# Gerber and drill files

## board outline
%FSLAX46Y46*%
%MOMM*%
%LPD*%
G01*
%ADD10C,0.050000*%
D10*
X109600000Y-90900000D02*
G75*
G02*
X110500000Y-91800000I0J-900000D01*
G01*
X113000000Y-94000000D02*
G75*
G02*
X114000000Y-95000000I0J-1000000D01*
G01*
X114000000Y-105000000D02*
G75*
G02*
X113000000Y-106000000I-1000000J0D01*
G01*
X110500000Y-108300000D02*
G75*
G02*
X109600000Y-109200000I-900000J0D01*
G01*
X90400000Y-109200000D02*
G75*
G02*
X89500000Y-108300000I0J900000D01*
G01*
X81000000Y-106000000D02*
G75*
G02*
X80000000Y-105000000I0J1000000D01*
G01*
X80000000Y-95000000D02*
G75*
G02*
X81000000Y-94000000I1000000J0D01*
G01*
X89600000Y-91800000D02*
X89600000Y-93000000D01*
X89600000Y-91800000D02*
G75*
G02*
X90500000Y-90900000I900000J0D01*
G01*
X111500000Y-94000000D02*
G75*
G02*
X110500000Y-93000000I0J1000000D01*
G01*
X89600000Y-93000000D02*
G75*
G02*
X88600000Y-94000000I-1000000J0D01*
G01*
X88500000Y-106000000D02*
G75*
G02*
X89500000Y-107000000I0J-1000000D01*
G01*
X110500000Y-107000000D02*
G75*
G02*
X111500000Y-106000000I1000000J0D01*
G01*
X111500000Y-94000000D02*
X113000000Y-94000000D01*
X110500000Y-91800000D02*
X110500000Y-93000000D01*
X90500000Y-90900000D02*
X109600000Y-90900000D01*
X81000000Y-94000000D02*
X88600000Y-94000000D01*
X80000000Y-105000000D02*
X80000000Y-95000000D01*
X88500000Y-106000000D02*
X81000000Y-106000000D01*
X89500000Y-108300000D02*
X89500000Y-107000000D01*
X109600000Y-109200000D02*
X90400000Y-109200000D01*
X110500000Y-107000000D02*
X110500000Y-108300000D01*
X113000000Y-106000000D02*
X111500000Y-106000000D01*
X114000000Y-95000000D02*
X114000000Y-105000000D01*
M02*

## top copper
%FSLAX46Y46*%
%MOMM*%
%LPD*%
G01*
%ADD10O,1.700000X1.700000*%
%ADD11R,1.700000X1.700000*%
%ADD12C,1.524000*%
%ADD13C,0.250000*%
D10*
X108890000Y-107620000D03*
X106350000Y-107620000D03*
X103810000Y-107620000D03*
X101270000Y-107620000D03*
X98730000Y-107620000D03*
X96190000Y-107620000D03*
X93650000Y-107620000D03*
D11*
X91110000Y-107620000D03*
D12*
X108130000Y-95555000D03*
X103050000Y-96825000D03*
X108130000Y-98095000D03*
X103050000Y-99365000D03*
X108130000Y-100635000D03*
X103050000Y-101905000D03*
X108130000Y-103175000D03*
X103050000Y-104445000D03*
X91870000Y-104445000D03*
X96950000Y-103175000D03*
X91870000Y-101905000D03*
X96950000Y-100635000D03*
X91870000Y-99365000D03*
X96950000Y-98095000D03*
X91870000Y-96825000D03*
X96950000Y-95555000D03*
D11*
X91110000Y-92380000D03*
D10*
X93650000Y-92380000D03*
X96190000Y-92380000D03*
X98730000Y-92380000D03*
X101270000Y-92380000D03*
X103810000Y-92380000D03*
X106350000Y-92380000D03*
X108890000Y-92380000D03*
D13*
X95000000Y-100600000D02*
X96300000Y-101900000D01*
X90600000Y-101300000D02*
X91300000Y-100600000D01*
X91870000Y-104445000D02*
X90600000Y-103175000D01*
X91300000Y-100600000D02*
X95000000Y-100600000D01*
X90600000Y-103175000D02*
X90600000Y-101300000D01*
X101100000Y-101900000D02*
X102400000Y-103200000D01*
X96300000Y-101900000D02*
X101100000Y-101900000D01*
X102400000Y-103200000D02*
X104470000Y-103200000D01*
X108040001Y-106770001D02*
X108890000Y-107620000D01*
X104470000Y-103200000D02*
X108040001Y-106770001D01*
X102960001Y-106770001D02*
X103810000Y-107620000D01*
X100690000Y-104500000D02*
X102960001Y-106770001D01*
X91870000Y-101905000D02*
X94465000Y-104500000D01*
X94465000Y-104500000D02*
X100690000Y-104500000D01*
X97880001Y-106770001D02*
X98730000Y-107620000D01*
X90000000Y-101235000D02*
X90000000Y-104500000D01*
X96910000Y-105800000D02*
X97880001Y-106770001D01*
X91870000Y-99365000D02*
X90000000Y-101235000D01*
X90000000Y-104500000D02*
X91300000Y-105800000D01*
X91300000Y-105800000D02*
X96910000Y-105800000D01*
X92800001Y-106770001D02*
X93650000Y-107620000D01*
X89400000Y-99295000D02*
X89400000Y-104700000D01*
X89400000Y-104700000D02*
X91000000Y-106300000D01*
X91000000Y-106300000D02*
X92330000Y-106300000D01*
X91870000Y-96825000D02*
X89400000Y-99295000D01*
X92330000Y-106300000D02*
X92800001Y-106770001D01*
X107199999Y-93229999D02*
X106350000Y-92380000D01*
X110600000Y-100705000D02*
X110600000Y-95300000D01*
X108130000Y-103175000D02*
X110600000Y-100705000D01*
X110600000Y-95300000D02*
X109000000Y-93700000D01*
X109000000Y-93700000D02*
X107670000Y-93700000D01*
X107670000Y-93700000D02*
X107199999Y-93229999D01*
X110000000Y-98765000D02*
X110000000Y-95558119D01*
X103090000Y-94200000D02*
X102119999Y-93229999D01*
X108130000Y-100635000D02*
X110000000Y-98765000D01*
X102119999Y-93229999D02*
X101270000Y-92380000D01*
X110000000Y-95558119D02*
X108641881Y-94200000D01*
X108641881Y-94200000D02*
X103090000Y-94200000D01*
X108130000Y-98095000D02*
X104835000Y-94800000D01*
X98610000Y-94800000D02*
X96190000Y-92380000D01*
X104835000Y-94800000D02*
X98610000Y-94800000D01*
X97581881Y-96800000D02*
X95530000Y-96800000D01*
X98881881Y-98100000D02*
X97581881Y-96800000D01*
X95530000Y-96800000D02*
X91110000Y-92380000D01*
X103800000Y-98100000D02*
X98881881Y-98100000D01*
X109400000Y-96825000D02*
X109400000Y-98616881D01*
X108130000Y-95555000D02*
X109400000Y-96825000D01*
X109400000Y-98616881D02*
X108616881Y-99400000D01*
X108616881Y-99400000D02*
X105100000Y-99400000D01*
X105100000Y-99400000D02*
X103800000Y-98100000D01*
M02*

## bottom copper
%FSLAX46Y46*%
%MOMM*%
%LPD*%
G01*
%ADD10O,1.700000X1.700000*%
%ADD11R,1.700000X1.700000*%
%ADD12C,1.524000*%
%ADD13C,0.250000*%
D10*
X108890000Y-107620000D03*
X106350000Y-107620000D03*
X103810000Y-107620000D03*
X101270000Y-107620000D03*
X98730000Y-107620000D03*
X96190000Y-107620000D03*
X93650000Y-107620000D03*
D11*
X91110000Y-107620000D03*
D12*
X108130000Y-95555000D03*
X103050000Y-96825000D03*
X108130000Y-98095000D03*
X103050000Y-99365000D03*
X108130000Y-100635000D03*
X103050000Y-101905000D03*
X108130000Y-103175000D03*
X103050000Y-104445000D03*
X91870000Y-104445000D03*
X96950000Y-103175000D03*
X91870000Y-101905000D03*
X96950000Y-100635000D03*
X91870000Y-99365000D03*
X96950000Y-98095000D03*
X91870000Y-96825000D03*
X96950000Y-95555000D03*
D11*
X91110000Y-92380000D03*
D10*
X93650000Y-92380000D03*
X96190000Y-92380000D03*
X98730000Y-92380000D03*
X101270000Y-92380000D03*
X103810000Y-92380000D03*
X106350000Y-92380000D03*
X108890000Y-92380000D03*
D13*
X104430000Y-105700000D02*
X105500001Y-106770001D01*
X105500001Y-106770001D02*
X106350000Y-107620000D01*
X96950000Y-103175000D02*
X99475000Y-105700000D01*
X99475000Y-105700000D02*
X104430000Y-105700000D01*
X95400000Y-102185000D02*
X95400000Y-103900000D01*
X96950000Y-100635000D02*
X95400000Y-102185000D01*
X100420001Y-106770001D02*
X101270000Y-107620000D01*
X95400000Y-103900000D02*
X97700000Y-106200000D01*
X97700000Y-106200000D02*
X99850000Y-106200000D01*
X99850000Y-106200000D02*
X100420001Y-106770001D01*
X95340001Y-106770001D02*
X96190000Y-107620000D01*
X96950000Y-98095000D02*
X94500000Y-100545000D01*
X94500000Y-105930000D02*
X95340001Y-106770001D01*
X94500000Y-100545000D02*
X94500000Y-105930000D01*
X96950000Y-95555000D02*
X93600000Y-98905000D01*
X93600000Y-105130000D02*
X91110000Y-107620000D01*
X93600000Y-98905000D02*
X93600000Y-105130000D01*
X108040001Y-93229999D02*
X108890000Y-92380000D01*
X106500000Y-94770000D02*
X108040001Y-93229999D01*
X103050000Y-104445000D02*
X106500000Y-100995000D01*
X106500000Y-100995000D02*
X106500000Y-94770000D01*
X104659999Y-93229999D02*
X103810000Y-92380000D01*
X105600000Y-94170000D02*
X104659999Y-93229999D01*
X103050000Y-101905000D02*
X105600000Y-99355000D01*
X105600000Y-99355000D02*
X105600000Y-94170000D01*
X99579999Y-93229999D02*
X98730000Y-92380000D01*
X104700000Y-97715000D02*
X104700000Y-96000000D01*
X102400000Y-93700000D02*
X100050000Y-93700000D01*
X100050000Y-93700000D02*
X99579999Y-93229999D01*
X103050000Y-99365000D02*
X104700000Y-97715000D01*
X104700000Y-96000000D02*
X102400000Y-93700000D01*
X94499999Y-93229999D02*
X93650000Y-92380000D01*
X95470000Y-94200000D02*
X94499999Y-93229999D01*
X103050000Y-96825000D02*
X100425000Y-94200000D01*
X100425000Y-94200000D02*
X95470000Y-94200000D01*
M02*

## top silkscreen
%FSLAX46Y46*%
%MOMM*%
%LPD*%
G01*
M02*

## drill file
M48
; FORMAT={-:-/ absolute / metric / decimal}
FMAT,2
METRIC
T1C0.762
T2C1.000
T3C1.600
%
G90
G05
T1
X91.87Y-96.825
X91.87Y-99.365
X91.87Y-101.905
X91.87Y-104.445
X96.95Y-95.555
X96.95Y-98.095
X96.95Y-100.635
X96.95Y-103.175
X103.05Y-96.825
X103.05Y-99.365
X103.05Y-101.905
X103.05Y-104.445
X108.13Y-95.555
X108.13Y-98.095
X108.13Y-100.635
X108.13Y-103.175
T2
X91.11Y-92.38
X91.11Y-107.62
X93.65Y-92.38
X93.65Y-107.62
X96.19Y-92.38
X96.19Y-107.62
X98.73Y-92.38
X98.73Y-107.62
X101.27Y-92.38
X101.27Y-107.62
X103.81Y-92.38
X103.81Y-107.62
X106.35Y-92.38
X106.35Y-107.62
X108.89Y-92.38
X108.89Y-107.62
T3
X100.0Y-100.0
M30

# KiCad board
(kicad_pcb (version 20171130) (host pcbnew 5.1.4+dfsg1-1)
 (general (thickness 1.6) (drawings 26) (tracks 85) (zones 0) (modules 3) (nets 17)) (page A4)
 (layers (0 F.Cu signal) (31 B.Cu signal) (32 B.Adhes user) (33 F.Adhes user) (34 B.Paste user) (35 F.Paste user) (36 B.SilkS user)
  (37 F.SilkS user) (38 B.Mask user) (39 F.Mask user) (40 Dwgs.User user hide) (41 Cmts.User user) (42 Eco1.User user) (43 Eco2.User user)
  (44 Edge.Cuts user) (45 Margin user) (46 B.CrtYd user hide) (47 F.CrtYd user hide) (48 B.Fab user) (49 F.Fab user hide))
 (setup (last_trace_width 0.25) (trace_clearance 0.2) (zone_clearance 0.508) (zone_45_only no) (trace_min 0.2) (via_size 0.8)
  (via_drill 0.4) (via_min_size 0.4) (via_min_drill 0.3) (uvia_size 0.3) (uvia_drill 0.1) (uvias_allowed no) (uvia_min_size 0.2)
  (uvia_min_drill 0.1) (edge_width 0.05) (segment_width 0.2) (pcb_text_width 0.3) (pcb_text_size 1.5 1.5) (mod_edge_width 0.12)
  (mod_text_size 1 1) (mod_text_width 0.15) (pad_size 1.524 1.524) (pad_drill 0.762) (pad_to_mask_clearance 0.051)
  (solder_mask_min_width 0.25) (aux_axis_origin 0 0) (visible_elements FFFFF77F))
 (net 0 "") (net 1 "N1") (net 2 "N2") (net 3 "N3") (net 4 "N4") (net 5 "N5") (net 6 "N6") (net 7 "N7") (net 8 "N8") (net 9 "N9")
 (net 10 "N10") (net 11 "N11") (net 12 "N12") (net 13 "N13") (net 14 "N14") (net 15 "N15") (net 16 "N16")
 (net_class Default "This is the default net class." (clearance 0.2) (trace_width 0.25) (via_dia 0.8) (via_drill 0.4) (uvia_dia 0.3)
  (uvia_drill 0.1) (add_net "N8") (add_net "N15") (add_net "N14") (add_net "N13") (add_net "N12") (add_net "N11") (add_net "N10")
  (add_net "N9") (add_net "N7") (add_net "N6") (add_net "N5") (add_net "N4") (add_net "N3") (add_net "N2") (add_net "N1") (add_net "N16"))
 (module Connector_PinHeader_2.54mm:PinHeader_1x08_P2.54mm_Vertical (layer B.Cu) (at 91.11 107.62 270)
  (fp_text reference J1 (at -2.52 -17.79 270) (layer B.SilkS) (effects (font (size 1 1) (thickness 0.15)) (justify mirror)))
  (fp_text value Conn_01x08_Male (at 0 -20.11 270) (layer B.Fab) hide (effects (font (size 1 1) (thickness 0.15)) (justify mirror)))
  (pad 8 thru_hole oval (at 0 -17.78 270) (size 1.7 1.7) (drill 1) (layers *.Cu *.Mask) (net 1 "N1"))
  (pad 7 thru_hole oval (at 0 -15.24 270) (size 1.7 1.7) (drill 1) (layers *.Cu *.Mask) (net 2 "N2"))
  (pad 6 thru_hole oval (at 0 -12.7 270) (size 1.7 1.7) (drill 1) (layers *.Cu *.Mask) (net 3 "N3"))
  (pad 5 thru_hole oval (at 0 -10.16 270) (size 1.7 1.7) (drill 1) (layers *.Cu *.Mask) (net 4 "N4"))
  (pad 4 thru_hole oval (at 0 -7.62 270) (size 1.7 1.7) (drill 1) (layers *.Cu *.Mask) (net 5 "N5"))
  (pad 3 thru_hole oval (at 0 -5.08 270) (size 1.7 1.7) (drill 1) (layers *.Cu *.Mask) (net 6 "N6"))
  (pad 2 thru_hole oval (at 0 -2.54 270) (size 1.7 1.7) (drill 1) (layers *.Cu *.Mask) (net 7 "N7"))
  (pad 1 thru_hole rect (at 0 0 270) (size 1.7 1.7) (drill 1) (layers *.Cu *.Mask) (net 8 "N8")))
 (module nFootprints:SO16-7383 (layer F.Cu) (at 100 100)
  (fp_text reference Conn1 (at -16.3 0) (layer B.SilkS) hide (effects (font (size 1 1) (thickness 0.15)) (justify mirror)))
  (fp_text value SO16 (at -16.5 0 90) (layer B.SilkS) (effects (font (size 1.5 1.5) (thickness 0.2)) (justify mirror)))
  (pad "" np_thru_hole circle (at 0 0) (size 1.6 1.6) (drill 1.6) (layers *.Cu *.Mask))
  (pad 16 thru_hole circle (at 8.13 -4.445) (size 1.524 1.524) (drill 0.762) (layers *.Cu *.Mask) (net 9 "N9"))
  (pad 15 thru_hole circle (at 3.05 -3.175) (size 1.524 1.524) (drill 0.762) (layers *.Cu *.Mask) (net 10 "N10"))
  (pad 14 thru_hole circle (at 8.13 -1.905) (size 1.524 1.524) (drill 0.762) (layers *.Cu *.Mask) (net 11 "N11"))
  (pad 13 thru_hole circle (at 3.05 -0.635) (size 1.524 1.524) (drill 0.762) (layers *.Cu *.Mask) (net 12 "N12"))
  (pad 12 thru_hole circle (at 8.13 0.635) (size 1.524 1.524) (drill 0.762) (layers *.Cu *.Mask) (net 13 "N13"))
  (pad 11 thru_hole circle (at 3.05 1.905) (size 1.524 1.524) (drill 0.762) (layers *.Cu *.Mask) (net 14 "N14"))
  (pad 10 thru_hole circle (at 8.13 3.175) (size 1.524 1.524) (drill 0.762) (layers *.Cu *.Mask) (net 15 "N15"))
  (pad 9 thru_hole circle (at 3.05 4.445) (size 1.524 1.524) (drill 0.762) (layers *.Cu *.Mask) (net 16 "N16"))
  (pad 8 thru_hole circle (at -8.13 4.445) (size 1.524 1.524) (drill 0.762) (layers *.Cu *.Mask) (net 1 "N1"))
  (pad 7 thru_hole circle (at -3.05 3.175) (size 1.524 1.524) (drill 0.762) (layers *.Cu *.Mask) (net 2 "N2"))
  (pad 6 thru_hole circle (at -8.13 1.905) (size 1.524 1.524) (drill 0.762) (layers *.Cu *.Mask) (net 3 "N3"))
  (pad 5 thru_hole circle (at -3.05 0.635) (size 1.524 1.524) (drill 0.762) (layers *.Cu *.Mask) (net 4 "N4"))
  (pad 4 thru_hole circle (at -8.13 -0.635) (size 1.524 1.524) (drill 0.762) (layers *.Cu *.Mask) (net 5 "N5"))
  (pad 3 thru_hole circle (at -3.05 -1.905) (size 1.524 1.524) (drill 0.762) (layers *.Cu *.Mask) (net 6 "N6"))
  (pad 2 thru_hole circle (at -8.13 -3.175) (size 1.524 1.524) (drill 0.762) (layers *.Cu *.Mask) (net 7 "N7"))
  (pad 1 thru_hole circle (at -3.05 -4.445) (size 1.524 1.524) (drill 0.762) (layers *.Cu *.Mask) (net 8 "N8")))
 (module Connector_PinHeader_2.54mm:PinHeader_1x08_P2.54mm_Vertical (layer B.Cu) (at 91.11 92.38 270)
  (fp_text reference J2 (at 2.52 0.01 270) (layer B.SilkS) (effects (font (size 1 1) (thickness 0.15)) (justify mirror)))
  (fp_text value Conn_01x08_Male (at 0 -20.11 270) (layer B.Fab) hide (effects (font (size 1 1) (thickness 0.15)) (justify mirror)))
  (pad 1 thru_hole rect (at 0 0 270) (size 1.7 1.7) (drill 1) (layers *.Cu *.Mask) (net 9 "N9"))
  (pad 2 thru_hole oval (at 0 -2.54 270) (size 1.7 1.7) (drill 1) (layers *.Cu *.Mask) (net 10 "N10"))
  (pad 3 thru_hole oval (at 0 -5.08 270) (size 1.7 1.7) (drill 1) (layers *.Cu *.Mask) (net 11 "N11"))
  (pad 4 thru_hole oval (at 0 -7.62 270) (size 1.7 1.7) (drill 1) (layers *.Cu *.Mask) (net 12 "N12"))
  (pad 5 thru_hole oval (at 0 -10.16 270) (size 1.7 1.7) (drill 1) (layers *.Cu *.Mask) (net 13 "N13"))
  (pad 6 thru_hole oval (at 0 -12.7 270) (size 1.7 1.7) (drill 1) (layers *.Cu *.Mask) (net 14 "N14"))
  (pad 7 thru_hole oval (at 0 -15.24 270) (size 1.7 1.7) (drill 1) (layers *.Cu *.Mask) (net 15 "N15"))
  (pad 8 thru_hole oval (at 0 -17.78 270) (size 1.7 1.7) (drill 1) (layers *.Cu *.Mask) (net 16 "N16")))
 (gr_arc (start 109.6 91.8) (end 110.5 91.8) (angle -90) (layer Edge.Cuts) (width 0.05))
 (gr_arc (start 113 95) (end 114 95) (angle -90) (layer Edge.Cuts) (width 0.05))
 (gr_arc (start 113 105) (end 113 106) (angle -90) (layer Edge.Cuts) (width 0.05))
 (gr_arc (start 109.6 108.3) (end 109.6 109.2) (angle -90) (layer Edge.Cuts) (width 0.05))
 (gr_arc (start 90.4 108.3) (end 89.5 108.3) (angle -90) (layer Edge.Cuts) (width 0.05))
 (gr_arc (start 81 105) (end 80 105) (angle -90) (layer Edge.Cuts) (width 0.05))
 (gr_arc (start 81 95) (end 81 94) (angle -90) (layer Edge.Cuts) (width 0.05))
 (gr_line (start 89.6 91.8) (end 89.6 93) (layer Edge.Cuts) (width 0.05))
 (gr_arc (start 90.5 91.8) (end 90.5 90.9) (angle -90) (layer Edge.Cuts) (width 0.05))
 (gr_arc (start 111.5 93) (end 110.5 93) (angle -90) (layer Edge.Cuts) (width 0.05))
 (gr_arc (start 88.6 93) (end 88.6 94) (angle -90) (layer Edge.Cuts) (width 0.05))
 (gr_arc (start 88.5 107) (end 89.5 107) (angle -90) (layer Edge.Cuts) (width 0.05))
 (gr_arc (start 111.5 107) (end 111.5 106) (angle -90) (layer Edge.Cuts) (width 0.05))
 (gr_line (start 111.5 94) (end 113 94) (layer Edge.Cuts) (width 0.05))
 (gr_line (start 110.5 91.8) (end 110.5 93) (layer Edge.Cuts) (width 0.05))
 (gr_line (start 90.5 90.9) (end 109.6 90.9) (layer Edge.Cuts) (width 0.05))
 (gr_line (start 81 94) (end 88.6 94) (layer Edge.Cuts) (width 0.05))
 (gr_line (start 80 105) (end 80 95) (layer Edge.Cuts) (width 0.05))
 (gr_line (start 88.5 106) (end 81 106) (layer Edge.Cuts) (width 0.05))
 (gr_line (start 89.5 108.3) (end 89.5 107) (layer Edge.Cuts) (width 0.05))
 (gr_line (start 109.6 109.2) (end 90.4 109.2) (layer Edge.Cuts) (width 0.05))
 (gr_line (start 110.5 107) (end 110.5 108.3) (layer Edge.Cuts) (width 0.05))
 (gr_line (start 113 106) (end 111.5 106) (layer Edge.Cuts) (width 0.05))
 (gr_line (start 114 95) (end 114 105) (layer Edge.Cuts) (width 0.05))
 (segment (start 95 100.6) (end 96.3 101.9) (width 0.25) (layer F.Cu) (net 1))
 (segment (start 90.6 101.3) (end 91.3 100.6) (width 0.25) (layer F.Cu) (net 1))
 (segment (start 91.87 104.445) (end 90.6 103.175) (width 0.25) (layer F.Cu) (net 1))
 (segment (start 91.3 100.6) (end 95 100.6) (width 0.25) (layer F.Cu) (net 1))
 (segment (start 90.6 103.175) (end 90.6 101.3) (width 0.25) (layer F.Cu) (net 1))
 (segment (start 101.1 101.9) (end 102.4 103.2) (width 0.25) (layer F.Cu) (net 1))
 (segment (start 96.3 101.9) (end 101.1 101.9) (width 0.25) (layer F.Cu) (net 1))
 (segment (start 102.4 103.2) (end 104.47 103.2) (width 0.25) (layer F.Cu) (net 1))
 (segment (start 108.040001 106.770001) (end 108.89 107.62) (width 0.25) (layer F.Cu) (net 1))
 (segment (start 104.47 103.2) (end 108.040001 106.770001) (width 0.25) (layer F.Cu) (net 1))
 (segment (start 104.43 105.7) (end 105.500001 106.770001) (width 0.25) (layer B.Cu) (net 2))
 (segment (start 105.500001 106.770001) (end 106.35 107.62) (width 0.25) (layer B.Cu) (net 2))
 (segment (start 96.95 103.175) (end 99.475 105.7) (width 0.25) (layer B.Cu) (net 2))
 (segment (start 99.475 105.7) (end 104.43 105.7) (width 0.25) (layer B.Cu) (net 2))
 (segment (start 102.960001 106.770001) (end 103.81 107.62) (width 0.25) (layer F.Cu) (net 3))
 (segment (start 100.69 104.5) (end 102.960001 106.770001) (width 0.25) (layer F.Cu) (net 3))
 (segment (start 91.87 101.905) (end 94.465 104.5) (width 0.25) (layer F.Cu) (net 3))
 (segment (start 94.465 104.5) (end 100.69 104.5) (width 0.25) (layer F.Cu) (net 3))
 (segment (start 95.4 102.185) (end 95.4 103.9) (width 0.25) (layer B.Cu) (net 4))
 (segment (start 96.95 100.635) (end 95.4 102.185) (width 0.25) (layer B.Cu) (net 4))
 (segment (start 100.420001 106.770001) (end 101.27 107.62) (width 0.25) (layer B.Cu) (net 4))
 (segment (start 95.4 103.9) (end 97.7 106.2) (width 0.25) (layer B.Cu) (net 4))
 (segment (start 97.7 106.2) (end 99.85 106.2) (width 0.25) (layer B.Cu) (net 4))
 (segment (start 99.85 106.2) (end 100.420001 106.770001) (width 0.25) (layer B.Cu) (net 4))
 (segment (start 97.880001 106.770001) (end 98.73 107.62) (width 0.25) (layer F.Cu) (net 5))
 (segment (start 90 101.235) (end 90 104.5) (width 0.25) (layer F.Cu) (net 5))
 (segment (start 96.91 105.8) (end 97.880001 106.770001) (width 0.25) (layer F.Cu) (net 5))
 (segment (start 91.87 99.365) (end 90 101.235) (width 0.25) (layer F.Cu) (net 5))
 (segment (start 90 104.5) (end 91.3 105.8) (width 0.25) (layer F.Cu) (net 5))
 (segment (start 91.3 105.8) (end 96.91 105.8) (width 0.25) (layer F.Cu) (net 5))
 (segment (start 95.340001 106.770001) (end 96.19 107.62) (width 0.25) (layer B.Cu) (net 6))
 (segment (start 96.95 98.095) (end 94.5 100.545) (width 0.25) (layer B.Cu) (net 6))
 (segment (start 94.5 105.93) (end 95.340001 106.770001) (width 0.25) (layer B.Cu) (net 6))
 (segment (start 94.5 100.545) (end 94.5 105.93) (width 0.25) (layer B.Cu) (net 6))
 (segment (start 92.800001 106.770001) (end 93.65 107.62) (width 0.25) (layer F.Cu) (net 7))
 (segment (start 89.4 99.295) (end 89.4 104.7) (width 0.25) (layer F.Cu) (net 7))
 (segment (start 89.4 104.7) (end 91 106.3) (width 0.25) (layer F.Cu) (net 7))
 (segment (start 91 106.3) (end 92.33 106.3) (width 0.25) (layer F.Cu) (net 7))
 (segment (start 91.87 96.825) (end 89.4 99.295) (width 0.25) (layer F.Cu) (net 7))
 (segment (start 92.33 106.3) (end 92.800001 106.770001) (width 0.25) (layer F.Cu) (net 7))
 (segment (start 96.95 95.555) (end 93.6 98.905) (width 0.25) (layer B.Cu) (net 8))
 (segment (start 93.6 105.13) (end 91.11 107.62) (width 0.25) (layer B.Cu) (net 8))
 (segment (start 93.6 98.905) (end 93.6 105.13) (width 0.25) (layer B.Cu) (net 8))
 (segment (start 108.040001 93.229999) (end 108.89 92.38) (width 0.25) (layer B.Cu) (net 16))
 (segment (start 106.5 94.77) (end 108.040001 93.229999) (width 0.25) (layer B.Cu) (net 16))
 (segment (start 103.05 104.445) (end 106.5 100.995) (width 0.25) (layer B.Cu) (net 16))
 (segment (start 106.5 100.995) (end 106.5 94.77) (width 0.25) (layer B.Cu) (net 16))
 (segment (start 107.199999 93.229999) (end 106.35 92.38) (width 0.25) (layer F.Cu) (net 15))
 (segment (start 110.6 100.705) (end 110.6 95.3) (width 0.25) (layer F.Cu) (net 15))
 (segment (start 108.13 103.175) (end 110.6 100.705) (width 0.25) (layer F.Cu) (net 15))
 (segment (start 110.6 95.3) (end 109 93.7) (width 0.25) (layer F.Cu) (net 15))
 (segment (start 109 93.7) (end 107.67 93.7) (width 0.25) (layer F.Cu) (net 15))
 (segment (start 107.67 93.7) (end 107.199999 93.229999) (width 0.25) (layer F.Cu) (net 15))
 (segment (start 104.659999 93.229999) (end 103.81 92.38) (width 0.25) (layer B.Cu) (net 14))
 (segment (start 105.6 94.17) (end 104.659999 93.229999) (width 0.25) (layer B.Cu) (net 14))
 (segment (start 103.05 101.905) (end 105.6 99.355) (width 0.25) (layer B.Cu) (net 14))
 (segment (start 105.6 99.355) (end 105.6 94.17) (width 0.25) (layer B.Cu) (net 14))
 (segment (start 110 98.765) (end 110 95.558119) (width 0.25) (layer F.Cu) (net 13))
 (segment (start 103.09 94.2) (end 102.119999 93.229999) (width 0.25) (layer F.Cu) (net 13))
 (segment (start 108.13 100.635) (end 110 98.765) (width 0.25) (layer F.Cu) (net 13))
 (segment (start 102.119999 93.229999) (end 101.27 92.38) (width 0.25) (layer F.Cu) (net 13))
 (segment (start 110 95.558119) (end 108.641881 94.2) (width 0.25) (layer F.Cu) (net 13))
 (segment (start 108.641881 94.2) (end 103.09 94.2) (width 0.25) (layer F.Cu) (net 13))
 (segment (start 99.579999 93.229999) (end 98.73 92.38) (width 0.25) (layer B.Cu) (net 12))
 (segment (start 104.7 97.715) (end 104.7 96) (width 0.25) (layer B.Cu) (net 12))
 (segment (start 102.4 93.7) (end 100.05 93.7) (width 0.25) (layer B.Cu) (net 12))
 (segment (start 100.05 93.7) (end 99.579999 93.229999) (width 0.25) (layer B.Cu) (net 12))
 (segment (start 103.05 99.365) (end 104.7 97.715) (width 0.25) (layer B.Cu) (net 12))
 (segment (start 104.7 96) (end 102.4 93.7) (width 0.25) (layer B.Cu) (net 12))
 (segment (start 108.13 98.095) (end 104.835 94.8) (width 0.25) (layer F.Cu) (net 11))
 (segment (start 98.61 94.8) (end 96.19 92.38) (width 0.25) (layer F.Cu) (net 11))
 (segment (start 104.835 94.8) (end 98.61 94.8) (width 0.25) (layer F.Cu) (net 11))
 (segment (start 94.499999 93.229999) (end 93.65 92.38) (width 0.25) (layer B.Cu) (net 10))
 (segment (start 95.47 94.2) (end 94.499999 93.229999) (width 0.25) (layer B.Cu) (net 10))
 (segment (start 103.05 96.825) (end 100.425 94.2) (width 0.25) (layer B.Cu) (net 10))
 (segment (start 100.425 94.2) (end 95.47 94.2) (width 0.25) (layer B.Cu) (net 10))
 (segment (start 97.581881 96.8) (end 95.53 96.8) (width 0.25) (layer F.Cu) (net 9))
 (segment (start 98.881881 98.1) (end 97.581881 96.8) (width 0.25) (layer F.Cu) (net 9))
 (segment (start 95.53 96.8) (end 91.11 92.38) (width 0.25) (layer F.Cu) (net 9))
 (segment (start 103.8 98.1) (end 98.881881 98.1) (width 0.25) (layer F.Cu) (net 9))
 (segment (start 109.4 96.825) (end 109.4 98.616881) (width 0.25) (layer F.Cu) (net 9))
 (segment (start 108.13 95.555) (end 109.4 96.825) (width 0.25) (layer F.Cu) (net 9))
 (segment (start 109.4 98.616881) (end 108.616881 99.4) (width 0.25) (layer F.Cu) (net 9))
 (segment (start 108.616881 99.4) (end 105.1 99.4) (width 0.25) (layer F.Cu) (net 9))
 (segment (start 105.1 99.4) (end 103.8 98.1) (width 0.25) (layer F.Cu) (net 9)))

